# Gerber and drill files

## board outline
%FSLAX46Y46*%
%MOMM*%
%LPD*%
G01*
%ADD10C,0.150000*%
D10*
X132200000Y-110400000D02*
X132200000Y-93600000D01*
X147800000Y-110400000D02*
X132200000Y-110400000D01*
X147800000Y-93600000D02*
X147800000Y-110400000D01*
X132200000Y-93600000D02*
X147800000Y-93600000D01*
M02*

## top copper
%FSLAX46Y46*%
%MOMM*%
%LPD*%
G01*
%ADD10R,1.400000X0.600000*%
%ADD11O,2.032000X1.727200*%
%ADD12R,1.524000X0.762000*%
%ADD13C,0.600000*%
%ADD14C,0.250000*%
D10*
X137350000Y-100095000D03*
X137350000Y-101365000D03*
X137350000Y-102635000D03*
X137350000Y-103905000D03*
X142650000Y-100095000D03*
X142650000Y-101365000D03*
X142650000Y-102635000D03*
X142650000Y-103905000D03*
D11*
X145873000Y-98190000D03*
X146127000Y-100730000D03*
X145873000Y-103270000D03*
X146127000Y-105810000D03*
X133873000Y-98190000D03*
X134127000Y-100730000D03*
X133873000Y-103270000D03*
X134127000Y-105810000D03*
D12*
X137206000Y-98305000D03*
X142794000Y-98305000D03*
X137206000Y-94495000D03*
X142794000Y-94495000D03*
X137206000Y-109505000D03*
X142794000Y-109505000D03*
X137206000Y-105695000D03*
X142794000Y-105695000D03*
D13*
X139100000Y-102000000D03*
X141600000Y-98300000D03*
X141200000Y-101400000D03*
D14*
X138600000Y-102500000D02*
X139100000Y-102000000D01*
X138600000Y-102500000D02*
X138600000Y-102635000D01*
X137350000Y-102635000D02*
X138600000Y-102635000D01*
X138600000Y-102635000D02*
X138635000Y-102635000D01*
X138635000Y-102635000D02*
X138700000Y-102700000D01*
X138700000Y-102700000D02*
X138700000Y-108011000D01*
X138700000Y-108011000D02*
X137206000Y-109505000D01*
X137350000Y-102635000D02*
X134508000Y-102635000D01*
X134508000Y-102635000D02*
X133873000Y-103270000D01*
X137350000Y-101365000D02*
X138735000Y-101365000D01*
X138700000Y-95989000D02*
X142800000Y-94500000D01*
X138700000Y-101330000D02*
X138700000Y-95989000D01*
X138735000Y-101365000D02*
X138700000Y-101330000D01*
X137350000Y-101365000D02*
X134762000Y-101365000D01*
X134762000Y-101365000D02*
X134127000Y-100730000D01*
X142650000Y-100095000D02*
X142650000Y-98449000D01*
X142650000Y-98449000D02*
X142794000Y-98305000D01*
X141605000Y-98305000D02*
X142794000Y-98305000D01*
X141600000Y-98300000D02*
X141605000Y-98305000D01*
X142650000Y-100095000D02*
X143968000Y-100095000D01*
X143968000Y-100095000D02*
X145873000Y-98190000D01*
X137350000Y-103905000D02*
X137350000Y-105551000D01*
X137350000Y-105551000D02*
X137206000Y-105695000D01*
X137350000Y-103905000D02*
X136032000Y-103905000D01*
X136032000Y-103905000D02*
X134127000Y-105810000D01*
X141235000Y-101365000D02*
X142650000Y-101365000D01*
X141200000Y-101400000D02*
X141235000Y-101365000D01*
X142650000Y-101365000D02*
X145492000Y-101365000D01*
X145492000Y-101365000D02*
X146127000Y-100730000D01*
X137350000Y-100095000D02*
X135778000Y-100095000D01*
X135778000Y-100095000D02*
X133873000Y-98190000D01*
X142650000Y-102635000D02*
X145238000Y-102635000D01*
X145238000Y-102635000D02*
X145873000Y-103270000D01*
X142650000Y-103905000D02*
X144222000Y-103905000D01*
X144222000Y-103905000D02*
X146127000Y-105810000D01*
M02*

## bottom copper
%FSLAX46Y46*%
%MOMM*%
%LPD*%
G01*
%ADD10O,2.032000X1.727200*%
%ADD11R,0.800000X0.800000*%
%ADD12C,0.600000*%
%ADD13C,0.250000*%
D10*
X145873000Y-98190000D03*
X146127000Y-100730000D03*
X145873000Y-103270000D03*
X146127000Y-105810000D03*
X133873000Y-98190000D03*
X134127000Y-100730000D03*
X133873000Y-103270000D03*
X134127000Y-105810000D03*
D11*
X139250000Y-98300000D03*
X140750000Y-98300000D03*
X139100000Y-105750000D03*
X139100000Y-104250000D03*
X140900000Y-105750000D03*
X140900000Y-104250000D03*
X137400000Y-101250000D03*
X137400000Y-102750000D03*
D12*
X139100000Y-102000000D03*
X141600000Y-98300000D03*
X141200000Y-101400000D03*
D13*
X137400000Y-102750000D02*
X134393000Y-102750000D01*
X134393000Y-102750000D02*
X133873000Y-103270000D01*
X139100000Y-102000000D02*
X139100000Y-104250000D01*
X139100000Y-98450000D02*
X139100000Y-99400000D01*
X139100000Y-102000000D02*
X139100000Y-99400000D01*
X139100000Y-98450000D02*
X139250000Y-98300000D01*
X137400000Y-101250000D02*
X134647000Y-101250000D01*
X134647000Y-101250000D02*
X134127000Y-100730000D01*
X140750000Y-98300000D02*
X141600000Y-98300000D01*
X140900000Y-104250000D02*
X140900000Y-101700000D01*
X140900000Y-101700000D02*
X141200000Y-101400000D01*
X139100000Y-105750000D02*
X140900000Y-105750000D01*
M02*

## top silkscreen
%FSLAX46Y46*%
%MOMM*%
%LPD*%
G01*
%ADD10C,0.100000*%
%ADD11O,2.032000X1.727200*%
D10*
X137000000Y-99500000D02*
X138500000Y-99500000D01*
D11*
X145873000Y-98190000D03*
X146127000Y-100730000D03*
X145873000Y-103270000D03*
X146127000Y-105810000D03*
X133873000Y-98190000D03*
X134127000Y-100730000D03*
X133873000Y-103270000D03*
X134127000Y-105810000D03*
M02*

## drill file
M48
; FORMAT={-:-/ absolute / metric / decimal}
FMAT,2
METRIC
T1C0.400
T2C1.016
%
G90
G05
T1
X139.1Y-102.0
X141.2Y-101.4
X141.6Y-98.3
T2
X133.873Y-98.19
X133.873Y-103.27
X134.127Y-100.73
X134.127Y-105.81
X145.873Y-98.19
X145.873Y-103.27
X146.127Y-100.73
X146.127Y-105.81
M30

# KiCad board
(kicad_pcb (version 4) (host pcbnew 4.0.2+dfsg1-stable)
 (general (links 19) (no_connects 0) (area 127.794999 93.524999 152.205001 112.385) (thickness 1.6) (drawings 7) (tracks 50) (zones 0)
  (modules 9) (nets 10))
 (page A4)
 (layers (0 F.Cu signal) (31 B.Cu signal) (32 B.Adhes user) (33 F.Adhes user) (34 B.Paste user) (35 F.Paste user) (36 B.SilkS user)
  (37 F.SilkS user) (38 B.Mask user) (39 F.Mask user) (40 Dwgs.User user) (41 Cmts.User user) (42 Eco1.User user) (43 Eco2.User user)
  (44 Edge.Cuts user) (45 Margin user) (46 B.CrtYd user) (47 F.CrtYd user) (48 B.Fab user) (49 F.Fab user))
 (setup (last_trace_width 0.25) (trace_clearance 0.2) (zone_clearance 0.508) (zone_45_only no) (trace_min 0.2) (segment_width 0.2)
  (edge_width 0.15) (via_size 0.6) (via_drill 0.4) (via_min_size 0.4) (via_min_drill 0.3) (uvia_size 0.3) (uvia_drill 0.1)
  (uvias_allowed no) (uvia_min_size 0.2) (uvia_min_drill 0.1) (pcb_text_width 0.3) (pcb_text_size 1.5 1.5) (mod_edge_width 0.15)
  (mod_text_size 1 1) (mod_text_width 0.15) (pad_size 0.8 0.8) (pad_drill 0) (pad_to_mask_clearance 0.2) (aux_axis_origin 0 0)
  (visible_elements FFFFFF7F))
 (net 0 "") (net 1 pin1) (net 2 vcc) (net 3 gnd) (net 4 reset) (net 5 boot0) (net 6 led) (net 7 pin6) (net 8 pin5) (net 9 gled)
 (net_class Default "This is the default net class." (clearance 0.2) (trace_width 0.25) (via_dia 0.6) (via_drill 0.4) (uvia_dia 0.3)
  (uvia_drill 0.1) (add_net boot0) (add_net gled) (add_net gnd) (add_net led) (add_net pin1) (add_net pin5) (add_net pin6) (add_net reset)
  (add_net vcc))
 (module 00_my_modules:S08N (layer F.Cu) (at 140 102)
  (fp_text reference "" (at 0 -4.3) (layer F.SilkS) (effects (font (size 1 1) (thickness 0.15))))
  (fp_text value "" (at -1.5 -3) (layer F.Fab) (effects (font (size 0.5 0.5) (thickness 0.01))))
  (fp_line (start -3 -2.5) (end -1.5 -2.5) (layer F.SilkS) (width 0.1))
  (pad 1 smd rect (at -2.65 -1.905) (size 1.4 0.6) (layers F.Cu F.Paste F.Mask) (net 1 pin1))
  (pad VCC smd rect (at -2.65 -0.635) (size 1.4 0.6) (layers F.Cu F.Paste F.Mask) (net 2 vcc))
  (pad GND smd rect (at -2.65 0.635) (size 1.4 0.6) (layers F.Cu F.Paste F.Mask) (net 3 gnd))
  (pad NRST smd rect (at -2.65 1.905) (size 1.4 0.6) (layers F.Cu F.Paste F.Mask) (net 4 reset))
  (pad BOOT smd rect (at 2.65 -1.905) (size 1.4 0.6) (layers F.Cu F.Paste F.Mask) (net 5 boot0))
  (pad PA13 smd rect (at 2.65 -0.635) (size 1.4 0.6) (layers F.Cu F.Paste F.Mask) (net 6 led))
  (pad 6 smd rect (at 2.65 0.635) (size 1.4 0.6) (layers F.Cu F.Paste F.Mask) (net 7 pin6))
  (pad 5 smd rect (at 2.65 1.905) (size 1.4 0.6) (layers F.Cu F.Paste F.Mask) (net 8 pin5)))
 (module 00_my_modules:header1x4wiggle (layer F.Cu) (at 146 102)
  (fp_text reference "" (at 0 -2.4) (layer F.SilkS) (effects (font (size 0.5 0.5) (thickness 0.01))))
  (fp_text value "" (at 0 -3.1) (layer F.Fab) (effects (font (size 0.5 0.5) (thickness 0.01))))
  (pad BOOT thru_hole oval (at -0.127 -3.81) (size 2.032 1.7272) (drill 1.016) (layers *.Cu *.Mask F.SilkS) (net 5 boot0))
  (pad LED thru_hole oval (at 0.127 -1.27) (size 2.032 1.7272) (drill 1.016) (layers *.Cu *.Mask F.SilkS) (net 6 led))
  (pad 6 thru_hole oval (at -0.127 1.27) (size 2.032 1.7272) (drill 1.016) (layers *.Cu *.Mask F.SilkS) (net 7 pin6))
  (pad 5 thru_hole oval (at 0.127 3.81) (size 2.032 1.7272) (drill 1.016) (layers *.Cu *.Mask F.SilkS) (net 8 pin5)))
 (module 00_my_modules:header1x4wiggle (layer F.Cu) (at 134 102)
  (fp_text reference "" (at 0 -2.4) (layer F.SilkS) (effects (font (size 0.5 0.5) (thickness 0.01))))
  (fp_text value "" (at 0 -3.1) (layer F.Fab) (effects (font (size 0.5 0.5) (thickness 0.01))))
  (pad 1 thru_hole oval (at -0.127 -3.81) (size 2.032 1.7272) (drill 1.016) (layers *.Cu *.Mask F.SilkS) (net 1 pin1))
  (pad VCC thru_hole oval (at 0.127 -1.27) (size 2.032 1.7272) (drill 1.016) (layers *.Cu *.Mask F.SilkS) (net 2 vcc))
  (pad GND thru_hole oval (at -0.127 1.27) (size 2.032 1.7272) (drill 1.016) (layers *.Cu *.Mask F.SilkS) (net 3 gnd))
  (pad NRST thru_hole oval (at 0.127 3.81) (size 2.032 1.7272) (drill 1.016) (layers *.Cu *.Mask F.SilkS) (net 4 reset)))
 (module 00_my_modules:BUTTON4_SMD (layer F.Cu) (at 140 96.4)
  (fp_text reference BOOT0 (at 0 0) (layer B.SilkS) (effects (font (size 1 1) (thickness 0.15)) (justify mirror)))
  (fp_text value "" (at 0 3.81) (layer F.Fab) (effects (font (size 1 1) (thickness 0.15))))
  (pad "" smd rect (at -2.794 1.905) (size 1.524 0.762) (layers F.Cu F.Paste F.Mask))
  (pad BOOT smd rect (at 2.794 1.905) (size 1.524 0.762) (layers F.Cu F.Paste F.Mask) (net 5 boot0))
  (pad "" smd rect (at -2.794 -1.905) (size 1.524 0.762) (layers F.Cu F.Paste F.Mask))
  (pad VCC smd rect (at 2.794 -1.905) (size 1.524 0.762) (layers F.Cu F.Paste F.Mask) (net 2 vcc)))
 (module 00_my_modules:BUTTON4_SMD (layer F.Cu) (at 140 107.6)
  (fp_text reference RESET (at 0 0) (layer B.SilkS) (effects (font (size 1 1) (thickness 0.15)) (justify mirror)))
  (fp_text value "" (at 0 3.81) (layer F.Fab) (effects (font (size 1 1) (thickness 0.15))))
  (pad GND smd rect (at -2.794 1.905) (size 1.524 0.762) (layers F.Cu F.Paste F.Mask) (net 3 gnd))
  (pad "" smd rect (at 2.794 1.905) (size 1.524 0.762) (layers F.Cu F.Paste F.Mask))
  (pad NRST smd rect (at -2.794 -1.905) (size 1.524 0.762) (layers F.Cu F.Paste F.Mask) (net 4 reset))
  (pad "" smd rect (at 2.794 -1.905) (size 1.524 0.762) (layers F.Cu F.Paste F.Mask)))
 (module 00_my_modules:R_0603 (layer B.Cu) (at 140 98.3)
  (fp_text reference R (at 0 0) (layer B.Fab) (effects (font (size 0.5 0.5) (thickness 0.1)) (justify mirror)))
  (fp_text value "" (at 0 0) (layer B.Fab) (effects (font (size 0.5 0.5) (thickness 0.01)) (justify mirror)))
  (pad GND smd rect (at -0.75 0) (size 0.8 0.8) (layers B.Cu B.Paste B.Mask) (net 3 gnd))
  (pad BOOT smd rect (at 0.75 0) (size 0.8 0.8) (layers B.Cu B.Paste B.Mask) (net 5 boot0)))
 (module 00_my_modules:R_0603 (layer B.Cu) (at 139.1 105 90)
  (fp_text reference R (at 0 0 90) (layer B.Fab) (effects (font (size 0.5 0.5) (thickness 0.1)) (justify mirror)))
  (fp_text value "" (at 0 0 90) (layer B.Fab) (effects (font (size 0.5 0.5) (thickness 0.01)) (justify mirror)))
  (pad GLED smd rect (at -0.75 0 90) (size 0.8 0.8) (layers B.Cu B.Paste B.Mask) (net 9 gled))
  (pad GND smd rect (at 0.75 0 90) (size 0.8 0.8) (layers B.Cu B.Paste B.Mask) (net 3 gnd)))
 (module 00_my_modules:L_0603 (layer B.Cu) (at 140.9 105 90)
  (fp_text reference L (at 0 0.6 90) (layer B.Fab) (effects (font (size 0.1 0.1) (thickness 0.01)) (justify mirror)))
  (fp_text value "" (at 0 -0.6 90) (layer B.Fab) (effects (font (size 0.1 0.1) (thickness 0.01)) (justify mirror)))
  (pad GLED smd rect (at -0.75 0 90) (size 0.8 0.8) (layers B.Cu B.Paste B.Mask) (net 9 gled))
  (pad LED smd rect (at 0.75 0 90) (size 0.8 0.8) (layers B.Cu B.Paste B.Mask) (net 6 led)))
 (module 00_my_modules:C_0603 (layer B.Cu) (at 137.4 102 270)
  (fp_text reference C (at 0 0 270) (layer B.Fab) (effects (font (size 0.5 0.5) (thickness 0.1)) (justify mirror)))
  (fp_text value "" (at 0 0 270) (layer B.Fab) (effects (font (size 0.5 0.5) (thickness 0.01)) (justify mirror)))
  (pad 1 smd rect (at -0.75 0 270) (size 0.8 0.8) (layers B.Cu B.Paste B.Mask) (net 2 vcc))
  (pad 2 smd rect (at 0.75 0 270) (size 0.8 0.8) (layers B.Cu B.Paste B.Mask) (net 3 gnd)))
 (gr_line (start 132.2 110.4) (end 132.2 93.6) (angle 90) (layer Edge.Cuts) (width 0.15))
 (gr_line (start 147.8 110.4) (end 132.2 110.4) (angle 90) (layer Edge.Cuts) (width 0.15))
 (gr_line (start 147.8 93.6) (end 147.8 110.4) (angle 90) (layer Edge.Cuts) (width 0.15))
 (gr_line (start 132.2 93.6) (end 147.8 93.6) (angle 90) (layer Edge.Cuts) (width 0.15))
 (segment (start 137.4 102.75) (end 134.393 102.75) (width 0.25) (layer B.Cu) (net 3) (status C00000))
 (segment (start 134.393 102.75) (end 133.873 103.27) (width 0.25) (layer B.Cu) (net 3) (status C00000))
 (segment (start 139.1 102) (end 139.1 104.25) (width 0.25) (layer B.Cu) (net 3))
 (segment (start 139.1 98.45) (end 139.1 99.4) (width 0.25) (layer B.Cu) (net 3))
 (segment (start 138.6 102.5) (end 139.1 102) (width 0.25) (layer F.Cu) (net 3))
 (via (at 139.1 102) (size 0.6) (drill 0.4) (layers F.Cu B.Cu) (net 3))
 (segment (start 139.1 102) (end 139.1 99.4) (width 0.25) (layer B.Cu) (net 3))
 (segment (start 138.6 102.5) (end 138.6 102.635) (width 0.25) (layer F.Cu) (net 3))
 (segment (start 139.1 98.45) (end 139.25 98.3) (width 0.25) (layer B.Cu) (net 3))
 (segment (start 137.35 102.635) (end 138.6 102.635) (width 0.25) (layer F.Cu) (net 3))
 (segment (start 138.6 102.635) (end 138.635 102.635) (width 0.25) (layer F.Cu) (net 3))
 (segment (start 138.635 102.635) (end 138.7 102.7) (width 0.25) (layer F.Cu) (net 3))
 (segment (start 138.7 102.7) (end 138.7 108.011) (width 0.25) (layer F.Cu) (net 3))
 (segment (start 138.7 108.011) (end 137.206 109.505) (width 0.25) (layer F.Cu) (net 3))
 (segment (start 137.35 102.635) (end 134.508 102.635) (width 0.25) (layer F.Cu) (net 3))
 (segment (start 134.508 102.635) (end 133.873 103.27) (width 0.25) (layer F.Cu) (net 3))
 (segment (start 137.4 101.25) (end 134.647 101.25) (width 0.25) (layer B.Cu) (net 2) (status C00000))
 (segment (start 134.647 101.25) (end 134.127 100.73) (width 0.25) (layer B.Cu) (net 2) (status C00000))
 (segment (start 137.35 101.365) (end 138.735 101.365) (width 0.25) (layer F.Cu) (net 2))
 (segment (start 138.7 95.989) (end 142.8 94.5) (width 0.25) (layer F.Cu) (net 2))
 (segment (start 138.7 101.33) (end 138.7 95.989) (width 0.25) (layer F.Cu) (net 2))
 (segment (start 138.735 101.365) (end 138.7 101.33) (width 0.25) (layer F.Cu) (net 2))
 (segment (start 137.35 101.365) (end 134.762 101.365) (width 0.25) (layer F.Cu) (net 2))
 (segment (start 134.762 101.365) (end 134.127 100.73) (width 0.25) (layer F.Cu) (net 2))
 (segment (start 142.65 100.095) (end 142.65 98.449) (width 0.25) (layer F.Cu) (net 5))
 (segment (start 142.65 98.449) (end 142.794 98.305) (width 0.25) (layer F.Cu) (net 5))
 (segment (start 140.75 98.3) (end 141.6 98.3) (width 0.25) (layer B.Cu) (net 5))
 (segment (start 141.605 98.305) (end 142.794 98.305) (width 0.25) (layer F.Cu) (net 5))
 (segment (start 141.6 98.3) (end 141.605 98.305) (width 0.25) (layer F.Cu) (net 5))
 (via (at 141.6 98.3) (size 0.6) (drill 0.4) (layers F.Cu B.Cu) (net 5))
 (segment (start 142.65 100.095) (end 143.968 100.095) (width 0.25) (layer F.Cu) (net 5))
 (segment (start 143.968 100.095) (end 145.873 98.19) (width 0.25) (layer F.Cu) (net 5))
 (segment (start 137.35 103.905) (end 137.35 105.551) (width 0.25) (layer F.Cu) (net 4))
 (segment (start 137.35 105.551) (end 137.206 105.695) (width 0.25) (layer F.Cu) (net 4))
 (segment (start 137.35 103.905) (end 136.032 103.905) (width 0.25) (layer F.Cu) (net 4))
 (segment (start 136.032 103.905) (end 134.127 105.81) (width 0.25) (layer F.Cu) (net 4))
 (segment (start 140.9 104.25) (end 140.9 101.7) (width 0.25) (layer B.Cu) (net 6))
 (segment (start 141.235 101.365) (end 142.65 101.365) (width 0.25) (layer F.Cu) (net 6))
 (segment (start 141.2 101.4) (end 141.235 101.365) (width 0.25) (layer F.Cu) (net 6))
 (via (at 141.2 101.4) (size 0.6) (drill 0.4) (layers F.Cu B.Cu) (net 6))
 (segment (start 140.9 101.7) (end 141.2 101.4) (width 0.25) (layer B.Cu) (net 6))
 (segment (start 142.65 101.365) (end 145.492 101.365) (width 0.25) (layer F.Cu) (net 6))
 (segment (start 145.492 101.365) (end 146.127 100.73) (width 0.25) (layer F.Cu) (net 6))
 (segment (start 139.1 105.75) (end 140.9 105.75) (width 0.25) (layer B.Cu) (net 9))
 (segment (start 137.35 100.095) (end 135.778 100.095) (width 0.25) (layer F.Cu) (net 1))
 (segment (start 135.778 100.095) (end 133.873 98.19) (width 0.25) (layer F.Cu) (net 1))
 (segment (start 142.65 102.635) (end 145.238 102.635) (width 0.25) (layer F.Cu) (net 7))
 (segment (start 145.238 102.635) (end 145.873 103.27) (width 0.25) (layer F.Cu) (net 7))
 (segment (start 142.65 103.905) (end 144.222 103.905) (width 0.25) (layer F.Cu) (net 8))
 (segment (start 144.222 103.905) (end 146.127 105.81) (width 0.25) (layer F.Cu) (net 8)))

